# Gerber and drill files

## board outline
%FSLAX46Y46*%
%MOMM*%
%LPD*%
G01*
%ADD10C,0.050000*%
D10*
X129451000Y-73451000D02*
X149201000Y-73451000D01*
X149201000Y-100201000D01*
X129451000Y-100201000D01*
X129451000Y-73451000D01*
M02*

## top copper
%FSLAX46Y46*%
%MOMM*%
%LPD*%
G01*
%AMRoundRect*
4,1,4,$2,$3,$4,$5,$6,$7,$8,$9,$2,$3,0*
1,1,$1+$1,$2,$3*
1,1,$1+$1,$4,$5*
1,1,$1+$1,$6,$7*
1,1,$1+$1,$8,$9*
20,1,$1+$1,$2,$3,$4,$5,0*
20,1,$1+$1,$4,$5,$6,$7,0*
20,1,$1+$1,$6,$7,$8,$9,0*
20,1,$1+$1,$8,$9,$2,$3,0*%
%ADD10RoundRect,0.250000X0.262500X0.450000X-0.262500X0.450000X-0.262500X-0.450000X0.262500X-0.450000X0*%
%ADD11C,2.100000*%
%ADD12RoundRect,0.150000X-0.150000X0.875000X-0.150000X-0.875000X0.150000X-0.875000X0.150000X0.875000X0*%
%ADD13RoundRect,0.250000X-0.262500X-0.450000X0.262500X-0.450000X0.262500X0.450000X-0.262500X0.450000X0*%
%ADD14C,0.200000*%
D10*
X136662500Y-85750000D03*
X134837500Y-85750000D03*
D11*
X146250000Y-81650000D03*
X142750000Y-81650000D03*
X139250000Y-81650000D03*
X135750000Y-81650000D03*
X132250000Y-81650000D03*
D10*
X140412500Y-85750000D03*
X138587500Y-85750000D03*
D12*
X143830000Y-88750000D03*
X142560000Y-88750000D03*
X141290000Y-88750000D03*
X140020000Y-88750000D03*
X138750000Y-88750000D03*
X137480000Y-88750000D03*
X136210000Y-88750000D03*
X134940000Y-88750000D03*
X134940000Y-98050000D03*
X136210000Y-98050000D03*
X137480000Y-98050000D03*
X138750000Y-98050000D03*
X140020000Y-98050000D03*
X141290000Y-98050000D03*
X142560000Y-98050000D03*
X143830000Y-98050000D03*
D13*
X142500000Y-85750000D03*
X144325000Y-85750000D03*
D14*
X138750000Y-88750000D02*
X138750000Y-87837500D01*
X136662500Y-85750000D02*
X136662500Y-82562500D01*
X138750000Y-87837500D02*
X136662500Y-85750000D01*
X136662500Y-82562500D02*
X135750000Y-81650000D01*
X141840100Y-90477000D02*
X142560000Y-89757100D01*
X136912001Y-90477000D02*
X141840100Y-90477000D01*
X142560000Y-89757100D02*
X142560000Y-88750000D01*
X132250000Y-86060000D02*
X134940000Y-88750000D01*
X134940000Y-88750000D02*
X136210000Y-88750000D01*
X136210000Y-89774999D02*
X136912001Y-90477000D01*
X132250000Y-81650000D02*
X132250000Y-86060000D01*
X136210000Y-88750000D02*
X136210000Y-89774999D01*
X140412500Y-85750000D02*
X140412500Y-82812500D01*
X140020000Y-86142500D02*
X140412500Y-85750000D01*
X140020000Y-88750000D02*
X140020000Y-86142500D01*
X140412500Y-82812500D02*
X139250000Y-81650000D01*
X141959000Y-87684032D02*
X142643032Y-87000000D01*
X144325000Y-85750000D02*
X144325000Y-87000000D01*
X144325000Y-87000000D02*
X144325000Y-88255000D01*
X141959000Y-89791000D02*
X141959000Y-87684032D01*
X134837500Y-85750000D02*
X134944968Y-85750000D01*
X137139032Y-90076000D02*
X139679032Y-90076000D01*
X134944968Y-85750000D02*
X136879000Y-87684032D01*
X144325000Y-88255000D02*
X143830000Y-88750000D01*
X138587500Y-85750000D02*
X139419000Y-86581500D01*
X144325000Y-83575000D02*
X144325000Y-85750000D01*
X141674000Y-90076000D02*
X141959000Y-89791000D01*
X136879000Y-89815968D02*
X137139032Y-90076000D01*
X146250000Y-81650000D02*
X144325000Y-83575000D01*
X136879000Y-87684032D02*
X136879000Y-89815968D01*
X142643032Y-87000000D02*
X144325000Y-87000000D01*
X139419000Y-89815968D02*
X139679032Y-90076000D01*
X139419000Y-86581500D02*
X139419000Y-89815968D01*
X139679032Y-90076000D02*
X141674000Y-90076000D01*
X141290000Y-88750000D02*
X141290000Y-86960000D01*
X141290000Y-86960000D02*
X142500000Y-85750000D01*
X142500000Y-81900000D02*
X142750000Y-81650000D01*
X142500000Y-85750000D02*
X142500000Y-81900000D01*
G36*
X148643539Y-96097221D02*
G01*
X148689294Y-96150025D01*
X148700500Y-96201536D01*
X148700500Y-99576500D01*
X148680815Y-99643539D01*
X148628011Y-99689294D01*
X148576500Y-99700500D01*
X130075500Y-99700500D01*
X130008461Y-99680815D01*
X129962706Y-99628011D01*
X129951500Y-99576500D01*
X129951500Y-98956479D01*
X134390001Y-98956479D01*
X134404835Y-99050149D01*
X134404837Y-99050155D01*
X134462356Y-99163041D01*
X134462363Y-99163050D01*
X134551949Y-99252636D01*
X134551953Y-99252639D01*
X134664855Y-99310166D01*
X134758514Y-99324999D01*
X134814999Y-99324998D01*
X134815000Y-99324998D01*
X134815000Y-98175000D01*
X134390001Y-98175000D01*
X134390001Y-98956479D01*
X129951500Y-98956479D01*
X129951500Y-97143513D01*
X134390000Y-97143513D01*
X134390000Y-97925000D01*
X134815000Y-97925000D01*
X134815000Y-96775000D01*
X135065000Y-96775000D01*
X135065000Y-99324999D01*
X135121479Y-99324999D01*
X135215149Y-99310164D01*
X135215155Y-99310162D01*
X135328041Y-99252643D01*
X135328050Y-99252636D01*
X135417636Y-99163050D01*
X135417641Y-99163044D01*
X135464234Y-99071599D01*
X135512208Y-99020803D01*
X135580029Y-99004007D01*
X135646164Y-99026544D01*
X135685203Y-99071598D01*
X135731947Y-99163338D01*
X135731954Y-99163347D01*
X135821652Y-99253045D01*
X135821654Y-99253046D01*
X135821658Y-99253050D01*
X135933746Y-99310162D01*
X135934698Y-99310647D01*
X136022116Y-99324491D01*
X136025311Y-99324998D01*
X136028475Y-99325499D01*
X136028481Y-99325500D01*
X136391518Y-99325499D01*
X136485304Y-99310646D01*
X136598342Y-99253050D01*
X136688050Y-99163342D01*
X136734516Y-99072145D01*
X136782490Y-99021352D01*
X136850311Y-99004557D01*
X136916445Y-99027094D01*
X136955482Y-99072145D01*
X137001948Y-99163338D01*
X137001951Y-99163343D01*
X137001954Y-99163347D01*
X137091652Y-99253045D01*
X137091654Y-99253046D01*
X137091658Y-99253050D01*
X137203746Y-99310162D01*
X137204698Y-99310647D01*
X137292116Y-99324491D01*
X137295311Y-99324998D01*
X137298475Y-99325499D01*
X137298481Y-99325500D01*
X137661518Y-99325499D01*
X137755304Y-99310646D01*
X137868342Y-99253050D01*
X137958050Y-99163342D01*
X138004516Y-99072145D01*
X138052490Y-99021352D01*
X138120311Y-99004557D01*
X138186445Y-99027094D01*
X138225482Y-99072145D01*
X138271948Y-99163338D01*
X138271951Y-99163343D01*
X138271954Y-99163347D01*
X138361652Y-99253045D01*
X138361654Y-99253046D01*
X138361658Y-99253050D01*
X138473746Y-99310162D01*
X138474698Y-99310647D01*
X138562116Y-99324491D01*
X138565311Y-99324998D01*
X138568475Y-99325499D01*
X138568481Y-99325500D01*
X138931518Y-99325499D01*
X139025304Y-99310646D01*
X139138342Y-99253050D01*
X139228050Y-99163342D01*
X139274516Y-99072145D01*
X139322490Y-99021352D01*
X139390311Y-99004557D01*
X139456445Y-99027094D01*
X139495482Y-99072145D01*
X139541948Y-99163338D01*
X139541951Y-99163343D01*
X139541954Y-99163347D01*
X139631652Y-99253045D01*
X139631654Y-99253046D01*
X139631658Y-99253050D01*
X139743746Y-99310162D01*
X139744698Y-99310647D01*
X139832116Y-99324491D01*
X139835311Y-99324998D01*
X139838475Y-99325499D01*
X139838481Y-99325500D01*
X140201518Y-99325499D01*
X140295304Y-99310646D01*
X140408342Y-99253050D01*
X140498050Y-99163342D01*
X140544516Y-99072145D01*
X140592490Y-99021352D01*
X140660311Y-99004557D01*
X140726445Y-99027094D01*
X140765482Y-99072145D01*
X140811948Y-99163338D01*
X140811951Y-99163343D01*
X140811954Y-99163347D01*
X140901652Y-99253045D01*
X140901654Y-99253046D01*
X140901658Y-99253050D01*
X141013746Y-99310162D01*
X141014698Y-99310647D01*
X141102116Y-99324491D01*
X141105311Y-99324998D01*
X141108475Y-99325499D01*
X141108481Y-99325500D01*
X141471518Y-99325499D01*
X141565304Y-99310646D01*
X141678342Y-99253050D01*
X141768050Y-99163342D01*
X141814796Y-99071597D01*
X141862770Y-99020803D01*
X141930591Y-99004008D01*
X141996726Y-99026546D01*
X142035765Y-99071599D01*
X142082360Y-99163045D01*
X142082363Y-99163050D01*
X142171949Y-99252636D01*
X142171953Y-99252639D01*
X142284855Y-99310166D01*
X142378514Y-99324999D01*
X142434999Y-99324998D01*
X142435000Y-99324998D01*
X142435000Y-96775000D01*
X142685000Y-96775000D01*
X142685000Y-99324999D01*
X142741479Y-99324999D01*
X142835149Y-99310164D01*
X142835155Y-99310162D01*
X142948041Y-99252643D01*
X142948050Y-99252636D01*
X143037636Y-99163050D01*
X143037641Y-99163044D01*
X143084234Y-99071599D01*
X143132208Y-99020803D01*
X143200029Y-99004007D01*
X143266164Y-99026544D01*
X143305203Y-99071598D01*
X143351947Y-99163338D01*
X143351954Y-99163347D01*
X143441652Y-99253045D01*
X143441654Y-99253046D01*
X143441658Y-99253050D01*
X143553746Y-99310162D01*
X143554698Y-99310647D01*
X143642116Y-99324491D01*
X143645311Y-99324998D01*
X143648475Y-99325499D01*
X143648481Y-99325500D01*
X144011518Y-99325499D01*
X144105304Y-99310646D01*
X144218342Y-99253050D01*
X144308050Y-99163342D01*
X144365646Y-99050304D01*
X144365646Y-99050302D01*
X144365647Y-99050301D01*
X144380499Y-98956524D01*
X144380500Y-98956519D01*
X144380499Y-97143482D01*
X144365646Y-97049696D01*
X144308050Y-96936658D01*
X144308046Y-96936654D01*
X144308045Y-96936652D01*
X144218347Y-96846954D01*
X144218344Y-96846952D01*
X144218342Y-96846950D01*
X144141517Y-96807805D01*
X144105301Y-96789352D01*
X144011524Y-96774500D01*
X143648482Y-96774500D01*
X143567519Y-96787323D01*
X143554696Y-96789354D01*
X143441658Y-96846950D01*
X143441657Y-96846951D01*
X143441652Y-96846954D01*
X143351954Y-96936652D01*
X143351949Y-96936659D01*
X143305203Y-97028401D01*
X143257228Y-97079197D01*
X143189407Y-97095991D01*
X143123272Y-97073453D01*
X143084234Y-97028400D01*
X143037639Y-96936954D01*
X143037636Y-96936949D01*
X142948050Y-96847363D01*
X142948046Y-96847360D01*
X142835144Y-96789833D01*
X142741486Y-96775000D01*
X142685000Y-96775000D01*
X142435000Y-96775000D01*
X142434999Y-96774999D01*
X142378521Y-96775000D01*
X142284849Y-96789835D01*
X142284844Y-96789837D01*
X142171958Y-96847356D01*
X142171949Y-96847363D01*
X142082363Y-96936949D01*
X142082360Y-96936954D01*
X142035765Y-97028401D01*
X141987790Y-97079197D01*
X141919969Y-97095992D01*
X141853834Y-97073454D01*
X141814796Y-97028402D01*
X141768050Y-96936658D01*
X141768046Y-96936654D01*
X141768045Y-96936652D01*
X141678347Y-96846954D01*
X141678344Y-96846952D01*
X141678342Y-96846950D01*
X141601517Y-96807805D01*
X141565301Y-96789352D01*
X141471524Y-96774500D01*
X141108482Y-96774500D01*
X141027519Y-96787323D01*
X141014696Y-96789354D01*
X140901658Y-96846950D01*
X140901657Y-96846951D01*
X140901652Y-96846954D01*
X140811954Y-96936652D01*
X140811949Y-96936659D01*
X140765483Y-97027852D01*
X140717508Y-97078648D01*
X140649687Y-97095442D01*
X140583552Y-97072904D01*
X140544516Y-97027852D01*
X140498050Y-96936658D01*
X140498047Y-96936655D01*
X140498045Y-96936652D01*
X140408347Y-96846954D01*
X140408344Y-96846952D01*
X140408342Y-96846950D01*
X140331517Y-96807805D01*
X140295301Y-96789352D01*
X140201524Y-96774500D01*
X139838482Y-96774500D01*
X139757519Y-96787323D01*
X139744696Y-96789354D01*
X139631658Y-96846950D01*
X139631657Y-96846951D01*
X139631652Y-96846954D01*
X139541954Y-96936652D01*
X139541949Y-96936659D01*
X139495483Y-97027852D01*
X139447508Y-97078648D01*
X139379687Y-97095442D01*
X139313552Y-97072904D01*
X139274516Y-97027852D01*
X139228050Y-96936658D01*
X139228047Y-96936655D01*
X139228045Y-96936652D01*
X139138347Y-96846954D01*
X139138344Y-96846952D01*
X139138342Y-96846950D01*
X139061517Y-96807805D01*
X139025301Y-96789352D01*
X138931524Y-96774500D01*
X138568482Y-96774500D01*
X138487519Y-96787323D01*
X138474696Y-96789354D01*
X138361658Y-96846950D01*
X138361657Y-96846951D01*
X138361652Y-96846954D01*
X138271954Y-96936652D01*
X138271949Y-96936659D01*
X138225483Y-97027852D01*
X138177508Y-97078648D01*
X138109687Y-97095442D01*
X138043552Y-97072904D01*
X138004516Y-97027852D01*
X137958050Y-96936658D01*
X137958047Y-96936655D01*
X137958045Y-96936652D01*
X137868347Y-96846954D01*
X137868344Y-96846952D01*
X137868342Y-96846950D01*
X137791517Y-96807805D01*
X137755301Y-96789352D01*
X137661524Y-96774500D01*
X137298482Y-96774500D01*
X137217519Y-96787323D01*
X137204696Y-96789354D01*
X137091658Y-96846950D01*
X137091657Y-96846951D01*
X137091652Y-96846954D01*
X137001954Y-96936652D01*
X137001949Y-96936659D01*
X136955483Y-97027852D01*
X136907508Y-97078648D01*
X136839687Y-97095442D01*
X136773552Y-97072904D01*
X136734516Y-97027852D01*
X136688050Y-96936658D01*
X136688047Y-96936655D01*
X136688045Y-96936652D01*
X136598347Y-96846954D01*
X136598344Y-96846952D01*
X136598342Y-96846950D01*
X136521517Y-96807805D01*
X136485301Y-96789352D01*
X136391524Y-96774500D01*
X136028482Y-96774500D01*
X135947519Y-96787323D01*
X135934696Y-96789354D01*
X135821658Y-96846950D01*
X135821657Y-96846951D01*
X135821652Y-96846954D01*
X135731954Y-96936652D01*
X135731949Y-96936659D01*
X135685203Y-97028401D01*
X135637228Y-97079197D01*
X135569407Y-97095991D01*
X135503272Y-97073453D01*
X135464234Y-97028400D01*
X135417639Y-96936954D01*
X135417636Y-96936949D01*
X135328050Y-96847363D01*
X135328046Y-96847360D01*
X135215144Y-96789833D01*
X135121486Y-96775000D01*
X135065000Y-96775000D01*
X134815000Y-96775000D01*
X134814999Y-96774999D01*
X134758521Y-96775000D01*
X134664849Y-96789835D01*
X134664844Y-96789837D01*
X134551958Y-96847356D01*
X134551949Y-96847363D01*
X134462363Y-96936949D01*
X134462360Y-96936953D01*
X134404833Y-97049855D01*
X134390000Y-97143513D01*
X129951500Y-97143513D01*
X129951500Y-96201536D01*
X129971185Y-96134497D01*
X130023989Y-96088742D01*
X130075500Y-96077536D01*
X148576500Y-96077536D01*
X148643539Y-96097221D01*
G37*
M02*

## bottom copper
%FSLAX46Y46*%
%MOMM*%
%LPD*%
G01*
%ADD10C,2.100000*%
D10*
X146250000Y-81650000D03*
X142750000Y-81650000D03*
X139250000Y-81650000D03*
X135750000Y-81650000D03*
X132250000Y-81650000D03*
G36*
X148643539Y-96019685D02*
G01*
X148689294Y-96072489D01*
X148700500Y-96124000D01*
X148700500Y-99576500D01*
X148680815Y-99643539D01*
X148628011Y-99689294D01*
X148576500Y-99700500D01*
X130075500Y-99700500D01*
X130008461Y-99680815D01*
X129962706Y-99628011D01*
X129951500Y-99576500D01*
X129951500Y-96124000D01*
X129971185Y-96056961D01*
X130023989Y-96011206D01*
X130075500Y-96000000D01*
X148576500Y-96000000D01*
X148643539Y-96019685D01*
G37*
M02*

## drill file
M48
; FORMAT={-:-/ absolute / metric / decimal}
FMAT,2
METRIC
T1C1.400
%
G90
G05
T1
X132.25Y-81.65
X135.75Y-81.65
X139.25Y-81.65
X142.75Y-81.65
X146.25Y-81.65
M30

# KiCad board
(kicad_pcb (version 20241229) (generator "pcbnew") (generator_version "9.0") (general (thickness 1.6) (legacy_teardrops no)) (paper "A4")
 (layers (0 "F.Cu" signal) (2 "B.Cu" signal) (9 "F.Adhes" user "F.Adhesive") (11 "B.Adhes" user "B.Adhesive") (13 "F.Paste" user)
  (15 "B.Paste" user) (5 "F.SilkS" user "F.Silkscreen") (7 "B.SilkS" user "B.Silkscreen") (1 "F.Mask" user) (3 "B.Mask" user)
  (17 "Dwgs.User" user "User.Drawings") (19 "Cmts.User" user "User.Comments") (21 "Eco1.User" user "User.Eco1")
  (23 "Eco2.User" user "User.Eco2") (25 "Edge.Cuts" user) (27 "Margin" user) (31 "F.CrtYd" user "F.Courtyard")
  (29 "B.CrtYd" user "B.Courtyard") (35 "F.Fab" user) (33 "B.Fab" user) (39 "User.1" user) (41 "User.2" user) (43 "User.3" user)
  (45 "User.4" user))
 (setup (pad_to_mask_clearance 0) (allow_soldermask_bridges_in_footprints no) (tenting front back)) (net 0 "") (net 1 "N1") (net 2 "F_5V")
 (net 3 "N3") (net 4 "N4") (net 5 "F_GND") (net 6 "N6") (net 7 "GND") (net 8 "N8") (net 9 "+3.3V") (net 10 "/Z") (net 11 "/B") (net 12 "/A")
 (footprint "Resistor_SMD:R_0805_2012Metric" (layer "F.Cu") (at 135.75 85.75 180)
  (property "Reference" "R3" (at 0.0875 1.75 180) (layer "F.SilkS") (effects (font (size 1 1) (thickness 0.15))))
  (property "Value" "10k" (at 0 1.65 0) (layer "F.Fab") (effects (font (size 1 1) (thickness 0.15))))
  (pad "1" smd roundrect (at -0.9125 0 180) (size 1.025 1.4) (layers "F.Cu" "F.Mask" "F.Paste") (roundrect_rratio 0.243902) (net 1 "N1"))
  (pad "2" smd roundrect (at 0.9125 0 180) (size 1.025 1.4) (layers "F.Cu" "F.Mask" "F.Paste") (roundrect_rratio 0.243902) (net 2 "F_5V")))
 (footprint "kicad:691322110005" (layer "F.Cu") (at 139.25 81.65 180)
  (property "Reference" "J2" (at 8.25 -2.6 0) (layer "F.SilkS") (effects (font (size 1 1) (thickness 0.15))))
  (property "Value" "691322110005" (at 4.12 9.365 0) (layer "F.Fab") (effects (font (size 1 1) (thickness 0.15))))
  (pad "1" thru_hole circle (at -7 0 180) (size 2.1 2.1) (drill 1.4) (layers "*.Cu" "*.Mask") (remove_unused_layers no) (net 2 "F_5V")
   (solder_mask_margin 0.102))
  (pad "2" thru_hole circle (at -3.5 0 180) (size 2.1 2.1) (drill 1.4) (layers "*.Cu" "*.Mask") (remove_unused_layers no) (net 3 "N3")
   (solder_mask_margin 0.102))
  (pad "3" thru_hole circle (at 0 0 180) (size 2.1 2.1) (drill 1.4) (layers "*.Cu" "*.Mask") (remove_unused_layers no) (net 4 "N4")
   (solder_mask_margin 0.102))
  (pad "4" thru_hole circle (at 3.5 0 180) (size 2.1 2.1) (drill 1.4) (layers "*.Cu" "*.Mask") (remove_unused_layers no) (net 1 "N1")
   (solder_mask_margin 0.102))
  (pad "5" thru_hole circle (at 7 0 180) (size 2.1 2.1) (drill 1.4) (layers "*.Cu" "*.Mask") (remove_unused_layers no) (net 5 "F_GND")
   (solder_mask_margin 0.102)))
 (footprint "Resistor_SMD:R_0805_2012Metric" (layer "F.Cu") (at 139.5 85.75 180)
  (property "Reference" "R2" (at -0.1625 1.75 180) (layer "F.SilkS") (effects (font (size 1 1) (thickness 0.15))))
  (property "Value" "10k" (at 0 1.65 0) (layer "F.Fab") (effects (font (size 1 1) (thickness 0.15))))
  (pad "1" smd roundrect (at -0.9125 0 180) (size 1.025 1.4) (layers "F.Cu" "F.Mask" "F.Paste") (roundrect_rratio 0.243902) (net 4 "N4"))
  (pad "2" smd roundrect (at 0.9125 0 180) (size 1.025 1.4) (layers "F.Cu" "F.Mask" "F.Paste") (roundrect_rratio 0.243902) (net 2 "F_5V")))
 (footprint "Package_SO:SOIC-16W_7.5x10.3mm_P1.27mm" (layer "F.Cu") (at 139.385 93.4 -90)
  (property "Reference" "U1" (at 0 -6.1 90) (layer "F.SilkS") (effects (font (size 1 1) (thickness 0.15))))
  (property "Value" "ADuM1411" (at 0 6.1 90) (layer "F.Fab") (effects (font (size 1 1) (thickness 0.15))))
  (pad "1" smd roundrect (at -4.65 -4.445 270) (size 2.05 0.6) (layers "F.Cu" "F.Mask" "F.Paste") (roundrect_rratio 0.25) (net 2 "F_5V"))
  (pad "2" smd roundrect (at -4.65 -3.175 270) (size 2.05 0.6) (layers "F.Cu" "F.Mask" "F.Paste") (roundrect_rratio 0.25) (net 5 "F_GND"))
  (pad "3" smd roundrect (at -4.65 -1.905 270) (size 2.05 0.6) (layers "F.Cu" "F.Mask" "F.Paste") (roundrect_rratio 0.25) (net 3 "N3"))
  (pad "4" smd roundrect (at -4.65 -0.635 270) (size 2.05 0.6) (layers "F.Cu" "F.Mask" "F.Paste") (roundrect_rratio 0.25) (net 4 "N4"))
  (pad "5" smd roundrect (at -4.65 0.635 270) (size 2.05 0.6) (layers "F.Cu" "F.Mask" "F.Paste") (roundrect_rratio 0.25) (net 1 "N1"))
  (pad "6" smd roundrect (at -4.65 1.905 270) (size 2.05 0.6) (layers "F.Cu" "F.Mask" "F.Paste") (roundrect_rratio 0.25) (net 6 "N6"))
  (pad "7" smd roundrect (at -4.65 3.175 270) (size 2.05 0.6) (layers "F.Cu" "F.Mask" "F.Paste") (roundrect_rratio 0.25) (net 5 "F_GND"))
  (pad "8" smd roundrect (at -4.65 4.445 270) (size 2.05 0.6) (layers "F.Cu" "F.Mask" "F.Paste") (roundrect_rratio 0.25) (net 5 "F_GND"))
  (pad "9" smd roundrect (at 4.65 4.445 270) (size 2.05 0.6) (layers "F.Cu" "F.Mask" "F.Paste") (roundrect_rratio 0.25) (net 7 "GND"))
  (pad "10" smd roundrect (at 4.65 3.175 270) (size 2.05 0.6) (layers "F.Cu" "F.Mask" "F.Paste") (roundrect_rratio 0.25) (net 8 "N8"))
  (pad "11" smd roundrect (at 4.65 1.905 270) (size 2.05 0.6) (layers "F.Cu" "F.Mask" "F.Paste") (roundrect_rratio 0.25) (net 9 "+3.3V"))
  (pad "12" smd roundrect (at 4.65 0.635 270) (size 2.05 0.6) (layers "F.Cu" "F.Mask" "F.Paste") (roundrect_rratio 0.25) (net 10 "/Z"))
  (pad "13" smd roundrect (at 4.65 -0.635 270) (size 2.05 0.6) (layers "F.Cu" "F.Mask" "F.Paste") (roundrect_rratio 0.25) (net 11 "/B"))
  (pad "14" smd roundrect (at 4.65 -1.905 270) (size 2.05 0.6) (layers "F.Cu" "F.Mask" "F.Paste") (roundrect_rratio 0.25) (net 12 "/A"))
  (pad "15" smd roundrect (at 4.65 -3.175 270) (size 2.05 0.6) (layers "F.Cu" "F.Mask" "F.Paste") (roundrect_rratio 0.25) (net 7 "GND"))
  (pad "16" smd roundrect (at 4.65 -4.445 270) (size 2.05 0.6) (layers "F.Cu" "F.Mask" "F.Paste") (roundrect_rratio 0.25) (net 9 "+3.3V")))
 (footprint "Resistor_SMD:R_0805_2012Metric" (layer "F.Cu") (at 143.4125 85.75)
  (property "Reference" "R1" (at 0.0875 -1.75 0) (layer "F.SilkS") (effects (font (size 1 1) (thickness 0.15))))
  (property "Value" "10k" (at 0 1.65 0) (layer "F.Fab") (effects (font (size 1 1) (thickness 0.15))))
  (pad "1" smd roundrect (at -0.9125 0) (size 1.025 1.4) (layers "F.Cu" "F.Mask" "F.Paste") (roundrect_rratio 0.243902) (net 3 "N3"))
  (pad "2" smd roundrect (at 0.9125 0) (size 1.025 1.4) (layers "F.Cu" "F.Mask" "F.Paste") (roundrect_rratio 0.243902) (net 2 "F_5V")))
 (gr_rect (start 129.451 73.451) (end 149.201 100.201) (stroke (width 0.05) (type default)) (fill no) (layer "Edge.Cuts"))
 (segment (start 138.75 88.75) (end 138.75 87.8375) (width 0.2) (layer "F.Cu") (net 1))
 (segment (start 136.6625 85.75) (end 136.6625 82.5625) (width 0.2) (layer "F.Cu") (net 1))
 (segment (start 138.75 87.8375) (end 136.6625 85.75) (width 0.2) (layer "F.Cu") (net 1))
 (segment (start 136.6625 82.5625) (end 135.75 81.65) (width 0.2) (layer "F.Cu") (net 1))
 (segment (start 141.8401 90.477) (end 142.56 89.7571) (width 0.2) (layer "F.Cu") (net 5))
 (segment (start 136.912001 90.477) (end 141.8401 90.477) (width 0.2) (layer "F.Cu") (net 5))
 (segment (start 142.56 89.7571) (end 142.56 88.75) (width 0.2) (layer "F.Cu") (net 5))
 (segment (start 132.25 86.06) (end 134.94 88.75) (width 0.2) (layer "F.Cu") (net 5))
 (segment (start 134.94 88.75) (end 136.21 88.75) (width 0.2) (layer "F.Cu") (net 5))
 (segment (start 136.21 89.774999) (end 136.912001 90.477) (width 0.2) (layer "F.Cu") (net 5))
 (segment (start 132.25 81.65) (end 132.25 86.06) (width 0.2) (layer "F.Cu") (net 5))
 (segment (start 136.21 88.75) (end 136.21 89.774999) (width 0.2) (layer "F.Cu") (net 5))
 (segment (start 140.4125 85.75) (end 140.4125 82.8125) (width 0.2) (layer "F.Cu") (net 4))
 (segment (start 140.02 86.1425) (end 140.4125 85.75) (width 0.2) (layer "F.Cu") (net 4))
 (segment (start 140.02 88.75) (end 140.02 86.1425) (width 0.2) (layer "F.Cu") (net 4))
 (segment (start 140.4125 82.8125) (end 139.25 81.65) (width 0.2) (layer "F.Cu") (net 4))
 (segment (start 141.959 87.684032) (end 142.643032 87) (width 0.2) (layer "F.Cu") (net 2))
 (segment (start 144.325 85.75) (end 144.325 87) (width 0.2) (layer "F.Cu") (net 2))
 (segment (start 144.325 87) (end 144.325 88.255) (width 0.2) (layer "F.Cu") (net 2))
 (segment (start 141.959 89.791) (end 141.959 87.684032) (width 0.2) (layer "F.Cu") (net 2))
 (segment (start 134.8375 85.75) (end 134.944968 85.75) (width 0.2) (layer "F.Cu") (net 2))
 (segment (start 137.139032 90.076) (end 139.679032 90.076) (width 0.2) (layer "F.Cu") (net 2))
 (segment (start 134.944968 85.75) (end 136.879 87.684032) (width 0.2) (layer "F.Cu") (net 2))
 (segment (start 144.325 88.255) (end 143.83 88.75) (width 0.2) (layer "F.Cu") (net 2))
 (segment (start 138.5875 85.75) (end 139.419 86.5815) (width 0.2) (layer "F.Cu") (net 2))
 (segment (start 144.325 83.575) (end 144.325 85.75) (width 0.2) (layer "F.Cu") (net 2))
 (segment (start 141.674 90.076) (end 141.959 89.791) (width 0.2) (layer "F.Cu") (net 2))
 (segment (start 136.879 89.815968) (end 137.139032 90.076) (width 0.2) (layer "F.Cu") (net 2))
 (segment (start 146.25 81.65) (end 144.325 83.575) (width 0.2) (layer "F.Cu") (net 2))
 (segment (start 136.879 87.684032) (end 136.879 89.815968) (width 0.2) (layer "F.Cu") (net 2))
 (segment (start 142.643032 87) (end 144.325 87) (width 0.2) (layer "F.Cu") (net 2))
 (segment (start 139.419 89.815968) (end 139.679032 90.076) (width 0.2) (layer "F.Cu") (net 2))
 (segment (start 139.419 86.5815) (end 139.419 89.815968) (width 0.2) (layer "F.Cu") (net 2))
 (segment (start 139.679032 90.076) (end 141.674 90.076) (width 0.2) (layer "F.Cu") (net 2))
 (segment (start 141.29 88.75) (end 141.29 86.96) (width 0.2) (layer "F.Cu") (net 3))
 (segment (start 141.29 86.96) (end 142.5 85.75) (width 0.2) (layer "F.Cu") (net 3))
 (segment (start 142.5 81.9) (end 142.75 81.65) (width 0.2) (layer "F.Cu") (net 3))
 (segment (start 142.5 85.75) (end 142.5 81.9) (width 0.2) (layer "F.Cu") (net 3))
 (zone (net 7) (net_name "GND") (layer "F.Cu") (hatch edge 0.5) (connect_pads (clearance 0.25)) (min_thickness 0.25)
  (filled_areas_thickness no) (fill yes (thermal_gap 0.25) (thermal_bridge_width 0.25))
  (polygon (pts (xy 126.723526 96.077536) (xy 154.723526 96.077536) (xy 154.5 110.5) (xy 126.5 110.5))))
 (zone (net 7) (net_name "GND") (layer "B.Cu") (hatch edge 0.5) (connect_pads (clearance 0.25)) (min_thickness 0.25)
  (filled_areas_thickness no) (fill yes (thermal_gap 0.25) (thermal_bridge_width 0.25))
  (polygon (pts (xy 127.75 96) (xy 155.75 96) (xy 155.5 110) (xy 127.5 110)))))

